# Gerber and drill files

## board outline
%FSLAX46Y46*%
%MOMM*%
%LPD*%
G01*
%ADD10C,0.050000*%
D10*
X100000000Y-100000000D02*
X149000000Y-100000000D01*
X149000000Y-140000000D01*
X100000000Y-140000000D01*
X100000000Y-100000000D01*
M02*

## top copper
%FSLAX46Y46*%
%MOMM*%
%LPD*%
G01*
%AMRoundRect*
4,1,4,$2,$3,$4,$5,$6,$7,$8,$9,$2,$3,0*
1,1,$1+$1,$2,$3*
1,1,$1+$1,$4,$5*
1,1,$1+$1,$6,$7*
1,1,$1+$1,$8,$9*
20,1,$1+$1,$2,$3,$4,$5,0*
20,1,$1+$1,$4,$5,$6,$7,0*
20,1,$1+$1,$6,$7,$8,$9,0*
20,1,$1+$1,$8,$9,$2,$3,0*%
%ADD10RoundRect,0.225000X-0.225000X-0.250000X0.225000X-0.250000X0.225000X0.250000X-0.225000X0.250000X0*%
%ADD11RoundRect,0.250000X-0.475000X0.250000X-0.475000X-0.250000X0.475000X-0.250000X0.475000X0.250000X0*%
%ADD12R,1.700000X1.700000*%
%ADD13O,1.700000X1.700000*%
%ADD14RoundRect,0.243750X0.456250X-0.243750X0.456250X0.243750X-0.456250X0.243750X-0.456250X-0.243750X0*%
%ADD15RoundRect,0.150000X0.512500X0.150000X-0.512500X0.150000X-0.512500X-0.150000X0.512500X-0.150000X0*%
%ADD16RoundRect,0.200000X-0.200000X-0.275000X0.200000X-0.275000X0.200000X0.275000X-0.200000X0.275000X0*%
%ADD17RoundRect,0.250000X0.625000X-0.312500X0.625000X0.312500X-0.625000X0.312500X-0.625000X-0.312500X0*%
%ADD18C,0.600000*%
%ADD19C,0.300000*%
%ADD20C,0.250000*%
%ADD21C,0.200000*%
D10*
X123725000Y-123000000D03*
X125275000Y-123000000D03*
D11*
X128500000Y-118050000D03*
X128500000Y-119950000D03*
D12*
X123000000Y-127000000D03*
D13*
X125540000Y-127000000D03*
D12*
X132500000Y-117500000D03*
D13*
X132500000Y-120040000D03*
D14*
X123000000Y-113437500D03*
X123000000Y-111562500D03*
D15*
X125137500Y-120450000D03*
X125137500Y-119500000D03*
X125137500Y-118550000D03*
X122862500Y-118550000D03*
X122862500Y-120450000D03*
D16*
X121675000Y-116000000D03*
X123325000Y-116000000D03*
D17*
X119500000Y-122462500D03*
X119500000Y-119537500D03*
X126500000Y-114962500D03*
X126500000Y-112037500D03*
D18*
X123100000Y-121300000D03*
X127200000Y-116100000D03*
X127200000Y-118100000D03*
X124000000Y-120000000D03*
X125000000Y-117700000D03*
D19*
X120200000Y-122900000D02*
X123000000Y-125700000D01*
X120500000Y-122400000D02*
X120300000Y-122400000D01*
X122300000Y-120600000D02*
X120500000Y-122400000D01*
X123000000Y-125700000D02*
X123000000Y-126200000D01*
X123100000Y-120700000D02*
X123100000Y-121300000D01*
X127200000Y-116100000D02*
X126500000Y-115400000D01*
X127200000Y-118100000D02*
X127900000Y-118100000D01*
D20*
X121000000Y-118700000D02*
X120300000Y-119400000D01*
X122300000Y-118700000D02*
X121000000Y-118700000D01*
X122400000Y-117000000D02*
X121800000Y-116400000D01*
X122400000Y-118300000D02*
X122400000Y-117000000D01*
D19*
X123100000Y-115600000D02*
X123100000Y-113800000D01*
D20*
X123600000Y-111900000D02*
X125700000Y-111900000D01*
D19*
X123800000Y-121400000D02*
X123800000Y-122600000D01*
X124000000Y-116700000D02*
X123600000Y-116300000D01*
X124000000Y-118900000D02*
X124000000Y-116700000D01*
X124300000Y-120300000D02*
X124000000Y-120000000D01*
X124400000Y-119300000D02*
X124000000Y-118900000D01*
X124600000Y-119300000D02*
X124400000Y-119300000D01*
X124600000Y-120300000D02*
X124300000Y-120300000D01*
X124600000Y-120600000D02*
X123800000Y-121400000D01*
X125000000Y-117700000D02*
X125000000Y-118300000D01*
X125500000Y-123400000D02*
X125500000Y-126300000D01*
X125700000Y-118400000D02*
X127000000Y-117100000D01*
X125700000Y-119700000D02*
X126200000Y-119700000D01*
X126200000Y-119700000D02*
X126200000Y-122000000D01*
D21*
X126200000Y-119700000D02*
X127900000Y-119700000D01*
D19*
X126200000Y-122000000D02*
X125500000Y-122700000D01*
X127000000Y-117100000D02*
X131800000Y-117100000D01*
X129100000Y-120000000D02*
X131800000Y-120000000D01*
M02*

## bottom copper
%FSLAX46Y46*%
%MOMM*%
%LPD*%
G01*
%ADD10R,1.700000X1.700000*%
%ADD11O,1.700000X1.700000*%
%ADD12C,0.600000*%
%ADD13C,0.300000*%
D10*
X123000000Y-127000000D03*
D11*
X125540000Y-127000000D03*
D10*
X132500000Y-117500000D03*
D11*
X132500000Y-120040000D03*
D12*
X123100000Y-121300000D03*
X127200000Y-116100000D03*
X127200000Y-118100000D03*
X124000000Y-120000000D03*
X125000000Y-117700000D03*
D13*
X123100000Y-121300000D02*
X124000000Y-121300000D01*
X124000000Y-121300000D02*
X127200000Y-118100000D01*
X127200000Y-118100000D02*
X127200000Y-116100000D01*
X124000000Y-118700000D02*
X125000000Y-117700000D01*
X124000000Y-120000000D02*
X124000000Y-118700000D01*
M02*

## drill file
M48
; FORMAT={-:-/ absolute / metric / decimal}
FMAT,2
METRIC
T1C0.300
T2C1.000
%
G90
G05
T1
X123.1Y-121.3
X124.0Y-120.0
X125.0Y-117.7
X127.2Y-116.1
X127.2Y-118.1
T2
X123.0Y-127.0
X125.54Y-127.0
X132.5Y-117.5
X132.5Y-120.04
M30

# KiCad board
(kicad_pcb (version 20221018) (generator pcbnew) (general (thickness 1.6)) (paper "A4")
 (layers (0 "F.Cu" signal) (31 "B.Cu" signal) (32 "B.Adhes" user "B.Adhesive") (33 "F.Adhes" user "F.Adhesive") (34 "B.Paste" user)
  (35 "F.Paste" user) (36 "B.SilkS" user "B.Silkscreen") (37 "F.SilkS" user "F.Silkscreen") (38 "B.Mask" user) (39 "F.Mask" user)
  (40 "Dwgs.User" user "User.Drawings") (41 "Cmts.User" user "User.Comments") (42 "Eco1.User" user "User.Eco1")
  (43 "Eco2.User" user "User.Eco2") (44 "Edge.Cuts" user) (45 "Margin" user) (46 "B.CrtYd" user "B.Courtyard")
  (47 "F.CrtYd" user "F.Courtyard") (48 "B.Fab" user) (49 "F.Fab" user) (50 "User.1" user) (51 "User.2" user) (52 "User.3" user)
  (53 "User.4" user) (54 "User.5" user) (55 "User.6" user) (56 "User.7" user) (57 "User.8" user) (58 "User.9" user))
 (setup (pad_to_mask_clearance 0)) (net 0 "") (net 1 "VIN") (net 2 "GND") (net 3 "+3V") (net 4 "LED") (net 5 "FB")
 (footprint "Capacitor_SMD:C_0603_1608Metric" (layer "F.Cu") (at 124.5 123)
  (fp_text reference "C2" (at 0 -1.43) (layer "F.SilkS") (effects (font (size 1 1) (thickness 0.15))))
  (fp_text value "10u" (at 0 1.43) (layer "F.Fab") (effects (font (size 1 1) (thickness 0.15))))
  (pad "1" smd roundrect (at -0.775 0) (size 0.9 0.95) (layers "F.Cu" "F.Paste" "F.Mask") (roundrect_rratio 0.25) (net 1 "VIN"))
  (pad "2" smd roundrect (at 0.775 0) (size 0.9 0.95) (layers "F.Cu" "F.Paste" "F.Mask") (roundrect_rratio 0.25) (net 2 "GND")))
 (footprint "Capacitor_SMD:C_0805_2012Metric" (layer "F.Cu") (at 128.5 119 -90)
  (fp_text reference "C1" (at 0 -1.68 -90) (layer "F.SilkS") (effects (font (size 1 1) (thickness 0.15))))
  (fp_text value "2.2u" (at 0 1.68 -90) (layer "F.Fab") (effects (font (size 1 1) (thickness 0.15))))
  (pad "1" smd roundrect (at -0.95 0 270) (size 1 1.45) (layers "F.Cu" "F.Paste" "F.Mask") (roundrect_rratio 0.25) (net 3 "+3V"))
  (pad "2" smd roundrect (at 0.95 0 270) (size 1 1.45) (layers "F.Cu" "F.Paste" "F.Mask") (roundrect_rratio 0.25) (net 2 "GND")))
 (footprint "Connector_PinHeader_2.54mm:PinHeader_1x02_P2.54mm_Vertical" (layer "F.Cu") (at 123 127 90)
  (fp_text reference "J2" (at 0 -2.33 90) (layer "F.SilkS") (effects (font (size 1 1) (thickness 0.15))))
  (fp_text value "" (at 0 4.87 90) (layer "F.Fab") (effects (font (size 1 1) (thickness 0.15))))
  (pad "1" thru_hole rect (at 0 0 90) (size 1.7 1.7) (drill 1) (layers "*.Cu" "*.Mask") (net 3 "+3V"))
  (pad "2" thru_hole oval (at 0 2.54 90) (size 1.7 1.7) (drill 1) (layers "*.Cu" "*.Mask") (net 2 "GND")))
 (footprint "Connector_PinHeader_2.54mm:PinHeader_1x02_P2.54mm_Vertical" (layer "F.Cu") (at 132.5 117.5)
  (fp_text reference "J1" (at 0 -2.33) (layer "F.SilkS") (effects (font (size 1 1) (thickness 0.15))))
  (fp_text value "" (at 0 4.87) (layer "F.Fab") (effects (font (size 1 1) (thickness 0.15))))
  (pad "1" thru_hole rect (at 0 0) (size 1.7 1.7) (drill 1) (layers "*.Cu" "*.Mask") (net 1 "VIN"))
  (pad "2" thru_hole oval (at 0 2.54) (size 1.7 1.7) (drill 1) (layers "*.Cu" "*.Mask") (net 2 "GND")))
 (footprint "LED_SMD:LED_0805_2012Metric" (layer "F.Cu") (at 123 112.5 90)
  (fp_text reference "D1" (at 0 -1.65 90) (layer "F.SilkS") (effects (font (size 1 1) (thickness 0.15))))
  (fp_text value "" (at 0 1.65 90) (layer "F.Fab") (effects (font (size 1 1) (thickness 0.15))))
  (pad "1" smd roundrect (at -0.9375 0 90) (size 0.975 1.4) (layers "F.Cu" "F.Paste" "F.Mask") (roundrect_rratio 0.25) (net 2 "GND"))
  (pad "2" smd roundrect (at 0.9375 0 90) (size 0.975 1.4) (layers "F.Cu" "F.Paste" "F.Mask") (roundrect_rratio 0.25) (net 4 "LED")))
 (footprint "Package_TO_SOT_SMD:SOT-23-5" (layer "F.Cu") (at 124 119.5 180)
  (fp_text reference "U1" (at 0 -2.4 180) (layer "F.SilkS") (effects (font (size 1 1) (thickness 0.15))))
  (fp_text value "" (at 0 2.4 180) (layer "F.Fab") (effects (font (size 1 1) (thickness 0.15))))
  (pad "1" smd roundrect (at -1.1375 -0.95 180) (size 1.325 0.6) (layers "F.Cu" "F.Paste" "F.Mask") (roundrect_rratio 0.25) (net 1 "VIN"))
  (pad "2" smd roundrect (at -1.1375 0 180) (size 1.325 0.6) (layers "F.Cu" "F.Paste" "F.Mask") (roundrect_rratio 0.25) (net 2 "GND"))
  (pad "3" smd roundrect (at -1.1375 0.95 180) (size 1.325 0.6) (layers "F.Cu" "F.Paste" "F.Mask") (roundrect_rratio 0.25) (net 1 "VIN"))
  (pad "4" smd roundrect (at 1.1375 0.95 180) (size 1.325 0.6) (layers "F.Cu" "F.Paste" "F.Mask") (roundrect_rratio 0.25) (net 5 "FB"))
  (pad "5" smd roundrect (at 1.1375 -0.95 180) (size 1.325 0.6) (layers "F.Cu" "F.Paste" "F.Mask") (roundrect_rratio 0.25) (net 3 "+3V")))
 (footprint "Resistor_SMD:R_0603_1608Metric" (layer "F.Cu") (at 122.5 116)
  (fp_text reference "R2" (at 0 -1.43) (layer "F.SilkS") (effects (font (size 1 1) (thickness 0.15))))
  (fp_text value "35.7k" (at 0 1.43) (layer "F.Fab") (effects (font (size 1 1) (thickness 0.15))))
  (pad "1" smd roundrect (at -0.825 0) (size 0.8 0.95) (layers "F.Cu" "F.Paste" "F.Mask") (roundrect_rratio 0.25) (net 5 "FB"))
  (pad "2" smd roundrect (at 0.825 0) (size 0.8 0.95) (layers "F.Cu" "F.Paste" "F.Mask") (roundrect_rratio 0.25) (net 2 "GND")))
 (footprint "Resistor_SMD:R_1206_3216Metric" (layer "F.Cu") (at 119.5 121 90)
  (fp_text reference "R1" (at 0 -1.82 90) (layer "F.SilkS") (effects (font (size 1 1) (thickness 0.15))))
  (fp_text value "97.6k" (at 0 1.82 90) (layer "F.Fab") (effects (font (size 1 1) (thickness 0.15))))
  (pad "1" smd roundrect (at -1.4625 0 90) (size 1.125 1.75) (layers "F.Cu" "F.Paste" "F.Mask") (roundrect_rratio 0.222222) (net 3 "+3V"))
  (pad "2" smd roundrect (at 1.4625 0 90) (size 1.125 1.75) (layers "F.Cu" "F.Paste" "F.Mask") (roundrect_rratio 0.222222) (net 5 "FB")))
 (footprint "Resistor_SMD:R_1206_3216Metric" (layer "F.Cu") (at 126.5 113.5 90)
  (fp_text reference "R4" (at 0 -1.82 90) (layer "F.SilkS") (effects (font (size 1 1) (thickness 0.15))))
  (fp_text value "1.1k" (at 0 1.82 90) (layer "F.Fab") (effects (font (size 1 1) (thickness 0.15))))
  (pad "1" smd roundrect (at -1.4625 0 90) (size 1.125 1.75) (layers "F.Cu" "F.Paste" "F.Mask") (roundrect_rratio 0.222222) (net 3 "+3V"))
  (pad "2" smd roundrect (at 1.4625 0 90) (size 1.125 1.75) (layers "F.Cu" "F.Paste" "F.Mask") (roundrect_rratio 0.222222) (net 4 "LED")))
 (gr_rect (start 100 100) (end 149 140) (stroke (width 0.05) (type default)) (fill none) (layer "Edge.Cuts"))
 (segment (start 120.2 122.9) (end 123 125.7) (width 0.3) (layer "F.Cu") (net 3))
 (segment (start 120.5 122.4) (end 120.3 122.4) (width 0.3) (layer "F.Cu") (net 3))
 (segment (start 122.3 120.6) (end 120.5 122.4) (width 0.3) (layer "F.Cu") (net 3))
 (segment (start 123 125.7) (end 123 126.2) (width 0.3) (layer "F.Cu") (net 3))
 (segment (start 123.1 120.7) (end 123.1 121.3) (width 0.3) (layer "F.Cu") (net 3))
 (segment (start 127.2 116.1) (end 126.5 115.4) (width 0.3) (layer "F.Cu") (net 3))
 (segment (start 127.2 118.1) (end 127.9 118.1) (width 0.3) (layer "F.Cu") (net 3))
 (via (at 123.1 121.3) (size 0.6) (drill 0.3) (layers "F.Cu" "B.Cu") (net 3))
 (via (at 127.2 116.1) (size 0.6) (drill 0.3) (layers "F.Cu" "B.Cu") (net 3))
 (via (at 127.2 118.1) (size 0.6) (drill 0.3) (layers "F.Cu" "B.Cu") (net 3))
 (segment (start 121 118.7) (end 120.3 119.4) (width 0.25) (layer "F.Cu") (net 5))
 (segment (start 122.3 118.7) (end 121 118.7) (width 0.25) (layer "F.Cu") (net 5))
 (segment (start 122.4 117) (end 121.8 116.4) (width 0.25) (layer "F.Cu") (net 5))
 (segment (start 122.4 118.3) (end 122.4 117) (width 0.25) (layer "F.Cu") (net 5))
 (segment (start 123.1 115.6) (end 123.1 113.8) (width 0.3) (layer "F.Cu") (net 2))
 (segment (start 123.1 121.3) (end 124 121.3) (width 0.3) (layer "B.Cu") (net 3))
 (segment (start 123.6 111.9) (end 125.7 111.9) (width 0.25) (layer "F.Cu") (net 4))
 (segment (start 123.8 121.4) (end 123.8 122.6) (width 0.3) (layer "F.Cu") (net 1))
 (segment (start 124 116.7) (end 123.6 116.3) (width 0.3) (layer "F.Cu") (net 2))
 (segment (start 124 118.9) (end 124 116.7) (width 0.3) (layer "F.Cu") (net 2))
 (segment (start 124 121.3) (end 127.2 118.1) (width 0.3) (layer "B.Cu") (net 3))
 (segment (start 124.3 120.3) (end 124 120) (width 0.3) (layer "F.Cu") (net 1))
 (segment (start 124.4 119.3) (end 124 118.9) (width 0.3) (layer "F.Cu") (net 2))
 (segment (start 124.6 119.3) (end 124.4 119.3) (width 0.3) (layer "F.Cu") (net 2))
 (segment (start 124.6 120.3) (end 124.3 120.3) (width 0.3) (layer "F.Cu") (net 1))
 (segment (start 124.6 120.6) (end 123.8 121.4) (width 0.3) (layer "F.Cu") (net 1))
 (segment (start 125 117.7) (end 125 118.3) (width 0.3) (layer "F.Cu") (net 1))
 (segment (start 125.5 123.4) (end 125.5 126.3) (width 0.3) (layer "F.Cu") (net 2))
 (segment (start 125.7 118.4) (end 127 117.1) (width 0.3) (layer "F.Cu") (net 1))
 (segment (start 125.7 119.7) (end 126.2 119.7) (width 0.3) (layer "F.Cu") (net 2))
 (segment (start 126.2 119.7) (end 126.2 122) (width 0.3) (layer "F.Cu") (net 2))
 (segment (start 126.2 119.7) (end 127.9 119.7) (width 0.2) (layer "F.Cu") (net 2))
 (segment (start 126.2 122) (end 125.5 122.7) (width 0.3) (layer "F.Cu") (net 2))
 (segment (start 127 117.1) (end 131.8 117.1) (width 0.3) (layer "F.Cu") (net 1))
 (segment (start 127.2 118.1) (end 127.2 116.1) (width 0.3) (layer "B.Cu") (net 3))
 (segment (start 129.1 120) (end 131.8 120) (width 0.3) (layer "F.Cu") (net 2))
 (via (at 124 120) (size 0.6) (drill 0.3) (layers "F.Cu" "B.Cu") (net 1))
 (via (at 125 117.7) (size 0.6) (drill 0.3) (layers "F.Cu" "B.Cu") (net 1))
 (segment (start 124 118.7) (end 125 117.7) (width 0.3) (layer "B.Cu") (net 1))
 (segment (start 124 120) (end 124 118.7) (width 0.3) (layer "B.Cu") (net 1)))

